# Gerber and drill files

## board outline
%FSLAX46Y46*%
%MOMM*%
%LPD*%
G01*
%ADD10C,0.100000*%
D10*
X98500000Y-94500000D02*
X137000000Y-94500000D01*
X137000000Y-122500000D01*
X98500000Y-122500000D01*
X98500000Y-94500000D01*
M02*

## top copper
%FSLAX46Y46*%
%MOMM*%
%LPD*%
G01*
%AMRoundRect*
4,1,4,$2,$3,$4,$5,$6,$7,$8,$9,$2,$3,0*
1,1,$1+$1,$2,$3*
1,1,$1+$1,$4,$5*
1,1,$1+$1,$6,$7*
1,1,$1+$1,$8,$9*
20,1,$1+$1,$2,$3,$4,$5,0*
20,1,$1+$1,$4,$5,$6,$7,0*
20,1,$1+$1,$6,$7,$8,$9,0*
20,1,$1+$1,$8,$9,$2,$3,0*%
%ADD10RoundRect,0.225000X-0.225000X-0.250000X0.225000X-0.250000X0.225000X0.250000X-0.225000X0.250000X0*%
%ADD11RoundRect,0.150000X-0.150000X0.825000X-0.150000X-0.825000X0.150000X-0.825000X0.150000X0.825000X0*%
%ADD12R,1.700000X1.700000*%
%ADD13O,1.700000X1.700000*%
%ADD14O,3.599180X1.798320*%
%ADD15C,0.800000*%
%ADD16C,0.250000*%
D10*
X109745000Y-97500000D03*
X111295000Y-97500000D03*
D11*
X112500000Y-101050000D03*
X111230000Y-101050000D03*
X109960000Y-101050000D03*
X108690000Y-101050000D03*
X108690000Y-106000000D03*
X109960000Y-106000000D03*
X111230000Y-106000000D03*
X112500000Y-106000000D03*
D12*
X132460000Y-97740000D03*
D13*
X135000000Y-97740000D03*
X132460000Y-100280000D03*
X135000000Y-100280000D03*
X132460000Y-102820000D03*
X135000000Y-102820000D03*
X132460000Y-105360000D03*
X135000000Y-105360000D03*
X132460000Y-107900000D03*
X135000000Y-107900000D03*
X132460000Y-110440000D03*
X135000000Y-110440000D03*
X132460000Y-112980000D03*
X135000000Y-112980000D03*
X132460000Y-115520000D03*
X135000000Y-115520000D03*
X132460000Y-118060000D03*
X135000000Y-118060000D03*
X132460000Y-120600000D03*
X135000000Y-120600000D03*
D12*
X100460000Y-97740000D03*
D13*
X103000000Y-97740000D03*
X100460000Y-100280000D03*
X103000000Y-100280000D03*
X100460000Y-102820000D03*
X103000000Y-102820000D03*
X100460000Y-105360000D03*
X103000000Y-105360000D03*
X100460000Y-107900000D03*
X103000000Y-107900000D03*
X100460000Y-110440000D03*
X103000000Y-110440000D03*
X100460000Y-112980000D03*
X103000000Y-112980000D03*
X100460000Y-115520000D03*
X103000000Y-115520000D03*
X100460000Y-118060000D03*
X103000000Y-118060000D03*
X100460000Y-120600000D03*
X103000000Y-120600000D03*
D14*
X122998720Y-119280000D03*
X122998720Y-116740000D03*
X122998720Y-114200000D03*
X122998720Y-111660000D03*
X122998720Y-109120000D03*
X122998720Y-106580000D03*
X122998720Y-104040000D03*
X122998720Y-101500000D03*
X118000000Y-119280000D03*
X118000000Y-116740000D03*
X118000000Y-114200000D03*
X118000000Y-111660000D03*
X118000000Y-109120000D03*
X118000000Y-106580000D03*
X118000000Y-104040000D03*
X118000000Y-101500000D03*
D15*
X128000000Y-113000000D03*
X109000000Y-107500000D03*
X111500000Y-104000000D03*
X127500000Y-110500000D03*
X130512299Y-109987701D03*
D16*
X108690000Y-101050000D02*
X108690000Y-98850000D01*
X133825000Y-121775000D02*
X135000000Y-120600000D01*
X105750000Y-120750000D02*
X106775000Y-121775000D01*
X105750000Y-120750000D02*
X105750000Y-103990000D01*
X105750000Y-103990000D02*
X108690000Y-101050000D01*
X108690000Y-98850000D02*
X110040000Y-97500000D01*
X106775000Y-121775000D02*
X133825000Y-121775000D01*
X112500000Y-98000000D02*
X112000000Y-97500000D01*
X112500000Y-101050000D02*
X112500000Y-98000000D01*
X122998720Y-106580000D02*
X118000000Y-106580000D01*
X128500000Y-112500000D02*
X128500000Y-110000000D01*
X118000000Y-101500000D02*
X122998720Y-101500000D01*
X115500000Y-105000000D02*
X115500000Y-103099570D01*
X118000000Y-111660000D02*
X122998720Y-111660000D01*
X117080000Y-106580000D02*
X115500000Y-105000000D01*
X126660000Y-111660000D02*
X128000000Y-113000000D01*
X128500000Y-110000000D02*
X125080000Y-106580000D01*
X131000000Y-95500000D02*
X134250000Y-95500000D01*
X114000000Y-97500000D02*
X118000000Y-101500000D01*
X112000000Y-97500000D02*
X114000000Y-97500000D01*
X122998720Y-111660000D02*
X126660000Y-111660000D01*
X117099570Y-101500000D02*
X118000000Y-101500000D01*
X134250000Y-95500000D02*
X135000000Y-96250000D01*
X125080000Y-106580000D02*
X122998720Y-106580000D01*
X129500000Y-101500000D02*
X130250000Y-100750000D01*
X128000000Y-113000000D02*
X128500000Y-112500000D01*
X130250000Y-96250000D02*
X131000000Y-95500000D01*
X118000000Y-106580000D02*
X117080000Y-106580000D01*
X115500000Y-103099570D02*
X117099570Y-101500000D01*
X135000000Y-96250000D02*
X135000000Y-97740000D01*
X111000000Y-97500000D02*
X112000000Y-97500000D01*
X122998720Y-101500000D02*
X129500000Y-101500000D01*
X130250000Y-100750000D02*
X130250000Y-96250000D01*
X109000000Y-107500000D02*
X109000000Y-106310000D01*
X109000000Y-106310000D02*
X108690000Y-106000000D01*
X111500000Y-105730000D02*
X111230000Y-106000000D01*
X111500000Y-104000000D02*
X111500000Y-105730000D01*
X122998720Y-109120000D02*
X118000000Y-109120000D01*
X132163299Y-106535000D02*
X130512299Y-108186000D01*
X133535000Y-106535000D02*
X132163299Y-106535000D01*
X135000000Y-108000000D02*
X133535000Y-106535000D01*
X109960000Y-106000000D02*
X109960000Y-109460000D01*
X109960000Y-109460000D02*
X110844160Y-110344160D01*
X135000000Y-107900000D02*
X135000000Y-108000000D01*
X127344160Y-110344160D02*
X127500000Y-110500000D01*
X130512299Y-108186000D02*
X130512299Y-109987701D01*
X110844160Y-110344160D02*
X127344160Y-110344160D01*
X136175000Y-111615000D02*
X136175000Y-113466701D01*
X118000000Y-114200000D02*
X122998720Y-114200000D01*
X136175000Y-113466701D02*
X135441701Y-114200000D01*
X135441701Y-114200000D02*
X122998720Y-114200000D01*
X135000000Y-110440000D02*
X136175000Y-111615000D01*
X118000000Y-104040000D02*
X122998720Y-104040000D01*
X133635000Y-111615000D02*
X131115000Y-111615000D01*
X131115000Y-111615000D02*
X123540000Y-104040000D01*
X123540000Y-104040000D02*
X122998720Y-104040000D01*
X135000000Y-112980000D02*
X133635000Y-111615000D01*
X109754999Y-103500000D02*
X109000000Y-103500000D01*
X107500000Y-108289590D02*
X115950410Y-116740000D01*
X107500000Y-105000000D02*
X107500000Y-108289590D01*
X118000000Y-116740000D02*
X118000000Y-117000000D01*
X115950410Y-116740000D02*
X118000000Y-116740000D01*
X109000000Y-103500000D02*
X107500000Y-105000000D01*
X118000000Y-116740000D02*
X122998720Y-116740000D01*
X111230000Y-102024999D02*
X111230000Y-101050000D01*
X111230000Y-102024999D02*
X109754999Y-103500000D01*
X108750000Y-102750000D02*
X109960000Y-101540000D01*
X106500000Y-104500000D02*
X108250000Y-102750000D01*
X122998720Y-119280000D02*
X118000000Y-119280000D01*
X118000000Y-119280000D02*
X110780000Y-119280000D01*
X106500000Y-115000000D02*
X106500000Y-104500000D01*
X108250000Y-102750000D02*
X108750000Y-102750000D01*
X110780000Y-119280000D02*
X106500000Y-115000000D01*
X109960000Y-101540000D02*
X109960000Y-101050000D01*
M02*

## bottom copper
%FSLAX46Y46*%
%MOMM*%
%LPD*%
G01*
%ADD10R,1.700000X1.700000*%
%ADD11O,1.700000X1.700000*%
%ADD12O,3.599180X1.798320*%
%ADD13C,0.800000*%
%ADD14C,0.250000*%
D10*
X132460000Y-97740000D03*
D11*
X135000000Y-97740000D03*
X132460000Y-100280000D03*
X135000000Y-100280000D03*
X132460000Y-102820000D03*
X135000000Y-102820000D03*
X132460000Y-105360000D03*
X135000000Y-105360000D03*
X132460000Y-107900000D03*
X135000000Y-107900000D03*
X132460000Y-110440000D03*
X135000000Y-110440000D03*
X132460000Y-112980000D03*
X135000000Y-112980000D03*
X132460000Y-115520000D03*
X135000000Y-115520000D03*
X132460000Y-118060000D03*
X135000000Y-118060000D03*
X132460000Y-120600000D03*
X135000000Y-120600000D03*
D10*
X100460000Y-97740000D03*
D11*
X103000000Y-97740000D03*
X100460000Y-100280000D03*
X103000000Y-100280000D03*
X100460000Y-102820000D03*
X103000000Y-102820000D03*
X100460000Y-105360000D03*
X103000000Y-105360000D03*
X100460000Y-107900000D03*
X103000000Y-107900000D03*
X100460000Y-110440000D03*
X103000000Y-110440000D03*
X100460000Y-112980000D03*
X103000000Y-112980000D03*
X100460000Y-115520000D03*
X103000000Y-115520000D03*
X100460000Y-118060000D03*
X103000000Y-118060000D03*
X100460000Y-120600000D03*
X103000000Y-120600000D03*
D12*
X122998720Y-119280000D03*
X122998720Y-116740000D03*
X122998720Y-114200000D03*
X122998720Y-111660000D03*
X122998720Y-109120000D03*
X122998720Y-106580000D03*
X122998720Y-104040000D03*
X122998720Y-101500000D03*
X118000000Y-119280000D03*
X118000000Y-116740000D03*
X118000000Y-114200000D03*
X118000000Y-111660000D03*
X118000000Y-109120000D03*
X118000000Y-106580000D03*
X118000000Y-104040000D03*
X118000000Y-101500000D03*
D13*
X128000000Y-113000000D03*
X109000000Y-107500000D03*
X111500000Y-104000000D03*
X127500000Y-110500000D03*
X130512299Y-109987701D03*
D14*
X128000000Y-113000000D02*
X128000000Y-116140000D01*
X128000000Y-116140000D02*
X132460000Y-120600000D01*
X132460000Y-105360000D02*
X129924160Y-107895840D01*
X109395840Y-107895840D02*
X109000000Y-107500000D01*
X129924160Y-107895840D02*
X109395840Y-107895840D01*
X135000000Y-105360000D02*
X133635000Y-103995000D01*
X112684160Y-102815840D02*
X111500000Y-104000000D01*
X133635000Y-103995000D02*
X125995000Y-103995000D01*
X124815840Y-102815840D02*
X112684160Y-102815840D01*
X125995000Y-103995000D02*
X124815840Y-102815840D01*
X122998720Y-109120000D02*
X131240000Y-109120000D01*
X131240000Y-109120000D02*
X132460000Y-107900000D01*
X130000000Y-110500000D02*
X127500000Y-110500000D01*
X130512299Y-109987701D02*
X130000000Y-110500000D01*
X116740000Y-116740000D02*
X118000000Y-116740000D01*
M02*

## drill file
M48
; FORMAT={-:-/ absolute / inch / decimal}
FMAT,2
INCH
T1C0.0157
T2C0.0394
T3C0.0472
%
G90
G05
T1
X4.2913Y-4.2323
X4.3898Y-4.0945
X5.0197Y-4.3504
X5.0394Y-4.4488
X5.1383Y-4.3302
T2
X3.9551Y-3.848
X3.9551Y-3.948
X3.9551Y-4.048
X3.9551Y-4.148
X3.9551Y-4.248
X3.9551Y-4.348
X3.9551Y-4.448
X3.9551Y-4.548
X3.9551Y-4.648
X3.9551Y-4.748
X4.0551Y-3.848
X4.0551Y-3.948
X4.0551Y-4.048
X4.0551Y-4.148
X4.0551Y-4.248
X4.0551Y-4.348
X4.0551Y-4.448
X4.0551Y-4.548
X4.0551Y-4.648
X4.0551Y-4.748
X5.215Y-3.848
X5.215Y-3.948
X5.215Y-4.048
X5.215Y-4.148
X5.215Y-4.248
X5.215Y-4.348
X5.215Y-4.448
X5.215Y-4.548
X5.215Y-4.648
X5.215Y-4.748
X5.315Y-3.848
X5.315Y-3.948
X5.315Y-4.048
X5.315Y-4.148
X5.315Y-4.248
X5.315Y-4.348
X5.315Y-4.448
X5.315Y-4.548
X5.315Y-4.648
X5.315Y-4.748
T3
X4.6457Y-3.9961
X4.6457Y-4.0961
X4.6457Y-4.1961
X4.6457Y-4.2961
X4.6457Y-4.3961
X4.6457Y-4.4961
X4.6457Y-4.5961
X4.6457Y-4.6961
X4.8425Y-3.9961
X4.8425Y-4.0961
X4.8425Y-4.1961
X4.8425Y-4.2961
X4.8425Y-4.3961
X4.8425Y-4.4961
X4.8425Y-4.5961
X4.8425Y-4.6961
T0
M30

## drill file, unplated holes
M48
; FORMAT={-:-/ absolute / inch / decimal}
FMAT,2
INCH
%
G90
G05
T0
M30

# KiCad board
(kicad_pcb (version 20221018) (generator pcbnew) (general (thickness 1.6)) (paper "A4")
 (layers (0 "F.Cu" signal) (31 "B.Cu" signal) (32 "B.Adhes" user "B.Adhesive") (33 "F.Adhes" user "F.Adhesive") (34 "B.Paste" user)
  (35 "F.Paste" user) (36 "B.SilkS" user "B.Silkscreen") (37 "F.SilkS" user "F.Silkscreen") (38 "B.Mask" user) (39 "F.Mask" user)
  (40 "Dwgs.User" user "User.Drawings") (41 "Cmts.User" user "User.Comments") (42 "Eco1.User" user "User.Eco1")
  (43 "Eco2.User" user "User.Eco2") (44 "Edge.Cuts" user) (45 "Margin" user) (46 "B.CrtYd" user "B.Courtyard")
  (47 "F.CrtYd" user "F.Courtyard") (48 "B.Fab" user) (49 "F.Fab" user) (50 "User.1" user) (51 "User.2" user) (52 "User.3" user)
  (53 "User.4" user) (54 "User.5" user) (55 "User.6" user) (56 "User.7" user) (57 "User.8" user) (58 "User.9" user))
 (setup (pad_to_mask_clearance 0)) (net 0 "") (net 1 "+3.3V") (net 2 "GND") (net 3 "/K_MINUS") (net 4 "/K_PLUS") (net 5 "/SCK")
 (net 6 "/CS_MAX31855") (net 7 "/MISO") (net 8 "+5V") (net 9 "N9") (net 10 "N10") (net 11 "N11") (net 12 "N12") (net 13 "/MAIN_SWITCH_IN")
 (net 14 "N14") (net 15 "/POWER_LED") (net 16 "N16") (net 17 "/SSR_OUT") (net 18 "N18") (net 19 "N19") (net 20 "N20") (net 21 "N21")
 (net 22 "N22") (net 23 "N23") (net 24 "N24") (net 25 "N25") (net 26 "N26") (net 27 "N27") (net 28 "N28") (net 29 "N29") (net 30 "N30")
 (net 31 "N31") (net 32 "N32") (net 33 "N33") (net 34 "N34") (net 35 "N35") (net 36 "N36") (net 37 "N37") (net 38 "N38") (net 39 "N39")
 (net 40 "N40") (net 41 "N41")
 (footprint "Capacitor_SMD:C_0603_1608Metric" (layer "F.Cu") (at 110.52 97.5)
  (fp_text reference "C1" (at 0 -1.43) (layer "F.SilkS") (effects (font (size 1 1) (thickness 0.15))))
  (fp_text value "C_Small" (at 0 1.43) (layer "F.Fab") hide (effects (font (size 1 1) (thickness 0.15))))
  (pad "1" smd roundrect (at -0.775 0) (size 0.9 0.95) (layers "F.Cu" "F.Paste" "F.Mask") (roundrect_rratio 0.25) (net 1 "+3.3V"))
  (pad "2" smd roundrect (at 0.775 0) (size 0.9 0.95) (layers "F.Cu" "F.Paste" "F.Mask") (roundrect_rratio 0.25) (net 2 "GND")))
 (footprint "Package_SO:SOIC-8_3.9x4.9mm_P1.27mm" (layer "F.Cu") (at 110.595 103.525 -90)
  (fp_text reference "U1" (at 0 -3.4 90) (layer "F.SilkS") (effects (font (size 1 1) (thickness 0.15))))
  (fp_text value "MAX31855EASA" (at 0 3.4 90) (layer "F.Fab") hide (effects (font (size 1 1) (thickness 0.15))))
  (pad "1" smd roundrect (at -2.475 -1.905 270) (size 1.95 0.6) (layers "F.Cu" "F.Paste" "F.Mask") (roundrect_rratio 0.25) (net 2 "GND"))
  (pad "2" smd roundrect (at -2.475 -0.635 270) (size 1.95 0.6) (layers "F.Cu" "F.Paste" "F.Mask") (roundrect_rratio 0.25)
   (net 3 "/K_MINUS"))
  (pad "3" smd roundrect (at -2.475 0.635 270) (size 1.95 0.6) (layers "F.Cu" "F.Paste" "F.Mask") (roundrect_rratio 0.25) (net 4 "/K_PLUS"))
  (pad "4" smd roundrect (at -2.475 1.905 270) (size 1.95 0.6) (layers "F.Cu" "F.Paste" "F.Mask") (roundrect_rratio 0.25) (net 1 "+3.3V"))
  (pad "5" smd roundrect (at 2.475 1.905 270) (size 1.95 0.6) (layers "F.Cu" "F.Paste" "F.Mask") (roundrect_rratio 0.25) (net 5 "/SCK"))
  (pad "6" smd roundrect (at 2.475 0.635 270) (size 1.95 0.6) (layers "F.Cu" "F.Paste" "F.Mask") (roundrect_rratio 0.25)
   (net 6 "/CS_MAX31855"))
  (pad "7" smd roundrect (at 2.475 -0.635 270) (size 1.95 0.6) (layers "F.Cu" "F.Paste" "F.Mask") (roundrect_rratio 0.25) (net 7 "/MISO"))
  (pad "8" smd roundrect (at 2.475 -1.905 270) (size 1.95 0.6) (layers "F.Cu" "F.Paste" "F.Mask") (roundrect_rratio 0.25)))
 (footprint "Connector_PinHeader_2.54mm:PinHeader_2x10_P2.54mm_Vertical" (layer "F.Cu") (at 132.46 97.74)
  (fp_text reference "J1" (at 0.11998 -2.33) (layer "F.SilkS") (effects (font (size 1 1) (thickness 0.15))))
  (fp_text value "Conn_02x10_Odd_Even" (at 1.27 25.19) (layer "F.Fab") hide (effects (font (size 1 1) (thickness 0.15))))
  (pad "1" thru_hole rect (at 0 0) (size 1.7 1.7) (drill 1) (layers "*.Cu" "*.Mask") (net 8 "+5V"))
  (pad "2" thru_hole oval (at 2.54 0) (size 1.7 1.7) (drill 1) (layers "*.Cu" "*.Mask") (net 2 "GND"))
  (pad "3" thru_hole oval (at 0 2.54) (size 1.7 1.7) (drill 1) (layers "*.Cu" "*.Mask") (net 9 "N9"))
  (pad "4" thru_hole oval (at 2.54 2.54) (size 1.7 1.7) (drill 1) (layers "*.Cu" "*.Mask") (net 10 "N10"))
  (pad "5" thru_hole oval (at 0 5.08) (size 1.7 1.7) (drill 1) (layers "*.Cu" "*.Mask") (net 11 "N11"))
  (pad "6" thru_hole oval (at 2.54 5.08) (size 1.7 1.7) (drill 1) (layers "*.Cu" "*.Mask") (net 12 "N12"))
  (pad "7" thru_hole oval (at 0 7.62) (size 1.7 1.7) (drill 1) (layers "*.Cu" "*.Mask") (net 5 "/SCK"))
  (pad "8" thru_hole oval (at 2.54 7.62) (size 1.7 1.7) (drill 1) (layers "*.Cu" "*.Mask") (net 7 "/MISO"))
  (pad "9" thru_hole oval (at 0 10.16) (size 1.7 1.7) (drill 1) (layers "*.Cu" "*.Mask") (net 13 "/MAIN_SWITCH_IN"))
  (pad "10" thru_hole oval (at 2.54 10.16) (size 1.7 1.7) (drill 1) (layers "*.Cu" "*.Mask") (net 6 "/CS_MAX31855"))
  (pad "11" thru_hole oval (at 0 12.7) (size 1.7 1.7) (drill 1) (layers "*.Cu" "*.Mask") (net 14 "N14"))
  (pad "12" thru_hole oval (at 2.54 12.7) (size 1.7 1.7) (drill 1) (layers "*.Cu" "*.Mask") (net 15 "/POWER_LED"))
  (pad "13" thru_hole oval (at 0 15.24) (size 1.7 1.7) (drill 1) (layers "*.Cu" "*.Mask") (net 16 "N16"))
  (pad "14" thru_hole oval (at 2.54 15.24) (size 1.7 1.7) (drill 1) (layers "*.Cu" "*.Mask") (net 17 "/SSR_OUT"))
  (pad "15" thru_hole oval (at 0 17.78) (size 1.7 1.7) (drill 1) (layers "*.Cu" "*.Mask") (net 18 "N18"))
  (pad "16" thru_hole oval (at 2.54 17.78) (size 1.7 1.7) (drill 1) (layers "*.Cu" "*.Mask") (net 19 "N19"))
  (pad "17" thru_hole oval (at 0 20.32) (size 1.7 1.7) (drill 1) (layers "*.Cu" "*.Mask") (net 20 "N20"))
  (pad "18" thru_hole oval (at 2.54 20.32) (size 1.7 1.7) (drill 1) (layers "*.Cu" "*.Mask") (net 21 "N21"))
  (pad "19" thru_hole oval (at 0 22.86) (size 1.7 1.7) (drill 1) (layers "*.Cu" "*.Mask") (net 2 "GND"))
  (pad "20" thru_hole oval (at 2.54 22.86) (size 1.7 1.7) (drill 1) (layers "*.Cu" "*.Mask") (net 1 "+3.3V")))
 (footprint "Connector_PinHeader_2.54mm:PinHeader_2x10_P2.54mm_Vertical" (layer "F.Cu") (at 100.46 97.74)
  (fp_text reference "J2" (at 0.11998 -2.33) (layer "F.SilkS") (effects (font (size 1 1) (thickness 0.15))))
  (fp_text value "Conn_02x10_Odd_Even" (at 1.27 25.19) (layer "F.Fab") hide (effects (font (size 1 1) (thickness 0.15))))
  (pad "1" thru_hole rect (at 0 0) (size 1.7 1.7) (drill 1) (layers "*.Cu" "*.Mask") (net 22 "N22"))
  (pad "2" thru_hole oval (at 2.54 0) (size 1.7 1.7) (drill 1) (layers "*.Cu" "*.Mask") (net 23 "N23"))
  (pad "3" thru_hole oval (at 0 2.54) (size 1.7 1.7) (drill 1) (layers "*.Cu" "*.Mask") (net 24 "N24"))
  (pad "4" thru_hole oval (at 2.54 2.54) (size 1.7 1.7) (drill 1) (layers "*.Cu" "*.Mask") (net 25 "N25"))
  (pad "5" thru_hole oval (at 0 5.08) (size 1.7 1.7) (drill 1) (layers "*.Cu" "*.Mask") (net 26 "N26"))
  (pad "6" thru_hole oval (at 2.54 5.08) (size 1.7 1.7) (drill 1) (layers "*.Cu" "*.Mask") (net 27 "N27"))
  (pad "7" thru_hole oval (at 0 7.62) (size 1.7 1.7) (drill 1) (layers "*.Cu" "*.Mask") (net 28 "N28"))
  (pad "8" thru_hole oval (at 2.54 7.62) (size 1.7 1.7) (drill 1) (layers "*.Cu" "*.Mask") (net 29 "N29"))
  (pad "9" thru_hole oval (at 0 10.16) (size 1.7 1.7) (drill 1) (layers "*.Cu" "*.Mask") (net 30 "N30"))
  (pad "10" thru_hole oval (at 2.54 10.16) (size 1.7 1.7) (drill 1) (layers "*.Cu" "*.Mask") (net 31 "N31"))
  (pad "11" thru_hole oval (at 0 12.7) (size 1.7 1.7) (drill 1) (layers "*.Cu" "*.Mask") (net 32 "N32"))
  (pad "12" thru_hole oval (at 2.54 12.7) (size 1.7 1.7) (drill 1) (layers "*.Cu" "*.Mask") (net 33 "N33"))
  (pad "13" thru_hole oval (at 0 15.24) (size 1.7 1.7) (drill 1) (layers "*.Cu" "*.Mask") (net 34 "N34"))
  (pad "14" thru_hole oval (at 2.54 15.24) (size 1.7 1.7) (drill 1) (layers "*.Cu" "*.Mask") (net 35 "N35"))
  (pad "15" thru_hole oval (at 0 17.78) (size 1.7 1.7) (drill 1) (layers "*.Cu" "*.Mask") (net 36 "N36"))
  (pad "16" thru_hole oval (at 2.54 17.78) (size 1.7 1.7) (drill 1) (layers "*.Cu" "*.Mask") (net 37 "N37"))
  (pad "17" thru_hole oval (at 0 20.32) (size 1.7 1.7) (drill 1) (layers "*.Cu" "*.Mask") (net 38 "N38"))
  (pad "18" thru_hole oval (at 2.54 20.32) (size 1.7 1.7) (drill 1) (layers "*.Cu" "*.Mask") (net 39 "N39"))
  (pad "19" thru_hole oval (at 0 22.86) (size 1.7 1.7) (drill 1) (layers "*.Cu" "*.Mask") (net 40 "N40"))
  (pad "20" thru_hole oval (at 2.54 22.86) (size 1.7 1.7) (drill 1) (layers "*.Cu" "*.Mask") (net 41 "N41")))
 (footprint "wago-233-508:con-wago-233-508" (layer "B.Cu") (at 120.49936 110.39 90)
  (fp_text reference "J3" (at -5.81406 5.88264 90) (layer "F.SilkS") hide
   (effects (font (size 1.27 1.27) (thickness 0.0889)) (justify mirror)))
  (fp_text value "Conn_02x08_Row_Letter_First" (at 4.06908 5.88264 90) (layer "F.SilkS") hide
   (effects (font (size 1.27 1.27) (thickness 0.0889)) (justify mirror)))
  (pad "a1" thru_hole oval (at -8.89 2.49936 90) (size 1.79832 3.59918) (drill 1.19888) (layers "*.Cu" "B.Paste" "B.Mask") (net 4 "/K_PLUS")
   (thermal_bridge_angle 45))
  (pad "a2" thru_hole oval (at -6.35 2.49936 90) (size 1.79832 3.59918) (drill 1.19888) (layers "*.Cu" "B.Paste" "B.Mask")
   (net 3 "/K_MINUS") (thermal_bridge_angle 45))
  (pad "a3" thru_hole oval (at -3.81 2.49936 90) (size 1.79832 3.59918) (drill 1.19888) (layers "*.Cu" "B.Paste" "B.Mask")
   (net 15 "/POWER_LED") (thermal_bridge_angle 45))
  (pad "a4" thru_hole oval (at -1.27 2.49936 90) (size 1.79832 3.59918) (drill 1.19888) (layers "*.Cu" "B.Paste" "B.Mask") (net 2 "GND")
   (thermal_bridge_angle 45))
  (pad "a5" thru_hole oval (at 1.27 2.49936 90) (size 1.79832 3.59918) (drill 1.19888) (layers "*.Cu" "B.Paste" "B.Mask")
   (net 13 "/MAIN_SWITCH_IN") (thermal_bridge_angle 45))
  (pad "a6" thru_hole oval (at 3.81 2.49936 90) (size 1.79832 3.59918) (drill 1.19888) (layers "*.Cu" "B.Paste" "B.Mask") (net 2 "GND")
   (thermal_bridge_angle 45))
  (pad "a7" thru_hole oval (at 6.35 2.49936 90) (size 1.79832 3.59918) (drill 1.19888) (layers "*.Cu" "B.Paste" "B.Mask")
   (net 17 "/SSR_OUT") (thermal_bridge_angle 45))
  (pad "a8" thru_hole oval (at 8.89 2.49936 90) (size 1.79832 3.59918) (drill 1.19888) (layers "*.Cu" "B.Paste" "B.Mask") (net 2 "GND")
   (thermal_bridge_angle 45))
  (pad "b1" thru_hole oval (at -8.89 -2.49936 90) (size 1.79832 3.59918) (drill 1.19888) (layers "*.Cu" "B.Paste" "B.Mask")
   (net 4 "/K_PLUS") (thermal_bridge_angle 45))
  (pad "b2" thru_hole oval (at -6.35 -2.49936 90) (size 1.79832 3.59918) (drill 1.19888) (layers "*.Cu" "B.Paste" "B.Mask")
   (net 3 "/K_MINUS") (thermal_bridge_angle 45))
  (pad "b3" thru_hole oval (at -3.81 -2.49936 90) (size 1.79832 3.59918) (drill 1.19888) (layers "*.Cu" "B.Paste" "B.Mask")
   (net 15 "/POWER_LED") (thermal_bridge_angle 45))
  (pad "b4" thru_hole oval (at -1.27 -2.49936 90) (size 1.79832 3.59918) (drill 1.19888) (layers "*.Cu" "B.Paste" "B.Mask") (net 2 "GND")
   (thermal_bridge_angle 45))
  (pad "b5" thru_hole oval (at 1.27 -2.49936 90) (size 1.79832 3.59918) (drill 1.19888) (layers "*.Cu" "B.Paste" "B.Mask")
   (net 13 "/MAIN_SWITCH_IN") (thermal_bridge_angle 45))
  (pad "b6" thru_hole oval (at 3.81 -2.49936 90) (size 1.79832 3.59918) (drill 1.19888) (layers "*.Cu" "B.Paste" "B.Mask") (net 2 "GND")
   (thermal_bridge_angle 45))
  (pad "b7" thru_hole oval (at 6.35 -2.49936 90) (size 1.79832 3.59918) (drill 1.19888) (layers "*.Cu" "B.Paste" "B.Mask")
   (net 17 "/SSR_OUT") (thermal_bridge_angle 45))
  (pad "b8" thru_hole oval (at 8.89 -2.49936 90) (size 1.79832 3.59918) (drill 1.19888) (layers "*.Cu" "B.Paste" "B.Mask") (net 2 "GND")
   (thermal_bridge_angle 45)))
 (gr_rect (start 98.5 94.5) (end 137 122.5) (stroke (width 0.1) (type default)) (fill none) (layer "Edge.Cuts"))
 (segment (start 108.69 101.05) (end 108.69 98.85) (width 0.25) (layer "F.Cu") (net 1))
 (segment (start 133.825 121.775) (end 135 120.6) (width 0.25) (layer "F.Cu") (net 1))
 (segment (start 105.75 120.75) (end 106.775 121.775) (width 0.25) (layer "F.Cu") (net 1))
 (segment (start 105.75 120.75) (end 105.75 103.99) (width 0.25) (layer "F.Cu") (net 1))
 (segment (start 105.75 103.99) (end 108.69 101.05) (width 0.25) (layer "F.Cu") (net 1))
 (segment (start 108.69 98.85) (end 110.04 97.5) (width 0.25) (layer "F.Cu") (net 1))
 (segment (start 106.775 121.775) (end 133.825 121.775) (width 0.25) (layer "F.Cu") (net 1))
 (segment (start 112.5 98) (end 112 97.5) (width 0.25) (layer "F.Cu") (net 2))
 (segment (start 112.5 101.05) (end 112.5 98) (width 0.25) (layer "F.Cu") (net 2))
 (segment (start 122.99872 106.58) (end 118 106.58) (width 0.25) (layer "F.Cu") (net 2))
 (segment (start 128.5 112.5) (end 128.5 110) (width 0.25) (layer "F.Cu") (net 2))
 (segment (start 118 101.5) (end 122.99872 101.5) (width 0.25) (layer "F.Cu") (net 2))
 (segment (start 115.5 105) (end 115.5 103.09957) (width 0.25) (layer "F.Cu") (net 2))
 (segment (start 118 111.66) (end 122.99872 111.66) (width 0.25) (layer "F.Cu") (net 2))
 (segment (start 117.08 106.58) (end 115.5 105) (width 0.25) (layer "F.Cu") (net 2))
 (segment (start 126.66 111.66) (end 128 113) (width 0.25) (layer "F.Cu") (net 2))
 (segment (start 128.5 110) (end 125.08 106.58) (width 0.25) (layer "F.Cu") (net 2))
 (segment (start 131 95.5) (end 134.25 95.5) (width 0.25) (layer "F.Cu") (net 2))
 (segment (start 114 97.5) (end 118 101.5) (width 0.25) (layer "F.Cu") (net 2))
 (segment (start 112 97.5) (end 114 97.5) (width 0.25) (layer "F.Cu") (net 2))
 (segment (start 122.99872 111.66) (end 126.66 111.66) (width 0.25) (layer "F.Cu") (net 2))
 (segment (start 117.09957 101.5) (end 118 101.5) (width 0.25) (layer "F.Cu") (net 2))
 (segment (start 134.25 95.5) (end 135 96.25) (width 0.25) (layer "F.Cu") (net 2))
 (segment (start 125.08 106.58) (end 122.99872 106.58) (width 0.25) (layer "F.Cu") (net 2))
 (segment (start 129.5 101.5) (end 130.25 100.75) (width 0.25) (layer "F.Cu") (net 2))
 (segment (start 128 113) (end 128.5 112.5) (width 0.25) (layer "F.Cu") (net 2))
 (segment (start 130.25 96.25) (end 131 95.5) (width 0.25) (layer "F.Cu") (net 2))
 (segment (start 118 106.58) (end 117.08 106.58) (width 0.25) (layer "F.Cu") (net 2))
 (segment (start 115.5 103.09957) (end 117.09957 101.5) (width 0.25) (layer "F.Cu") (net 2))
 (segment (start 135 96.25) (end 135 97.74) (width 0.25) (layer "F.Cu") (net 2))
 (segment (start 111 97.5) (end 112 97.5) (width 0.25) (layer "F.Cu") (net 2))
 (segment (start 122.99872 101.5) (end 129.5 101.5) (width 0.25) (layer "F.Cu") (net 2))
 (segment (start 130.25 100.75) (end 130.25 96.25) (width 0.25) (layer "F.Cu") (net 2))
 (via (at 128 113) (size 0.8) (drill 0.4) (layers "F.Cu" "B.Cu") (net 2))
 (segment (start 128 113) (end 128 116.14) (width 0.25) (layer "B.Cu") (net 2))
 (segment (start 128 116.14) (end 132.46 120.6) (width 0.25) (layer "B.Cu") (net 2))
 (segment (start 109 107.5) (end 109 106.31) (width 0.25) (layer "F.Cu") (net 5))
 (segment (start 109 106.31) (end 108.69 106) (width 0.25) (layer "F.Cu") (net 5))
 (via (at 109 107.5) (size 0.8) (drill 0.4) (layers "F.Cu" "B.Cu") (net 5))
 (segment (start 132.46 105.36) (end 129.92416 107.89584) (width 0.25) (layer "B.Cu") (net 5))
 (segment (start 109.39584 107.89584) (end 109 107.5) (width 0.25) (layer "B.Cu") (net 5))
 (segment (start 129.92416 107.89584) (end 109.39584 107.89584) (width 0.25) (layer "B.Cu") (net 5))
 (segment (start 111.5 105.73) (end 111.23 106) (width 0.25) (layer "F.Cu") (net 7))
 (segment (start 111.5 104) (end 111.5 105.73) (width 0.25) (layer "F.Cu") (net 7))
 (via (at 111.5 104) (size 0.8) (drill 0.4) (layers "F.Cu" "B.Cu") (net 7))
 (segment (start 135 105.36) (end 133.635 103.995) (width 0.25) (layer "B.Cu") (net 7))
 (segment (start 112.68416 102.81584) (end 111.5 104) (width 0.25) (layer "B.Cu") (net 7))
 (segment (start 133.635 103.995) (end 125.995 103.995) (width 0.25) (layer "B.Cu") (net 7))
 (segment (start 124.81584 102.81584) (end 112.68416 102.81584) (width 0.25) (layer "B.Cu") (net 7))
 (segment (start 125.995 103.995) (end 124.81584 102.81584) (width 0.25) (layer "B.Cu") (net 7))
 (segment (start 122.99872 109.12) (end 118 109.12) (width 0.25) (layer "F.Cu") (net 13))
 (segment (start 122.99872 109.12) (end 131.24 109.12) (width 0.25) (layer "B.Cu") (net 13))
 (segment (start 131.24 109.12) (end 132.46 107.9) (width 0.25) (layer "B.Cu") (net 13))
 (segment (start 132.163299 106.535) (end 130.512299 108.186) (width 0.25) (layer "F.Cu") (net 6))
 (segment (start 133.535 106.535) (end 132.163299 106.535) (width 0.25) (layer "F.Cu") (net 6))
 (segment (start 135 108) (end 133.535 106.535) (width 0.25) (layer "F.Cu") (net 6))
 (segment (start 109.96 106) (end 109.96 109.46) (width 0.25) (layer "F.Cu") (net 6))
 (segment (start 109.96 109.46) (end 110.84416 110.34416) (width 0.25) (layer "F.Cu") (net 6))
 (segment (start 135 107.9) (end 135 108) (width 0.25) (layer "F.Cu") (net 6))
 (segment (start 127.34416 110.34416) (end 127.5 110.5) (width 0.25) (layer "F.Cu") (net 6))
 (segment (start 130.512299 108.186) (end 130.512299 109.987701) (width 0.25) (layer "F.Cu") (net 6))
 (segment (start 110.84416 110.34416) (end 127.34416 110.34416) (width 0.25) (layer "F.Cu") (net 6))
 (via (at 127.5 110.5) (size 0.8) (drill 0.4) (layers "F.Cu" "B.Cu") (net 6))
 (via (at 130.512299 109.987701) (size 0.8) (drill 0.4) (layers "F.Cu" "B.Cu") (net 6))
 (segment (start 130 110.5) (end 127.5 110.5) (width 0.25) (layer "B.Cu") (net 6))
 (segment (start 130.512299 109.987701) (end 130 110.5) (width 0.25) (layer "B.Cu") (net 6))
 (segment (start 136.175 111.615) (end 136.175 113.466701) (width 0.25) (layer "F.Cu") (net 15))
 (segment (start 118 114.2) (end 122.99872 114.2) (width 0.25) (layer "F.Cu") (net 15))
 (segment (start 136.175 113.466701) (end 135.441701 114.2) (width 0.25) (layer "F.Cu") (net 15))
 (segment (start 135.441701 114.2) (end 122.99872 114.2) (width 0.25) (layer "F.Cu") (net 15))
 (segment (start 135 110.44) (end 136.175 111.615) (width 0.25) (layer "F.Cu") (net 15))
 (segment (start 118 104.04) (end 122.99872 104.04) (width 0.25) (layer "F.Cu") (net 17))
 (segment (start 133.635 111.615) (end 131.115 111.615) (width 0.25) (layer "F.Cu") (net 17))
 (segment (start 131.115 111.615) (end 123.54 104.04) (width 0.25) (layer "F.Cu") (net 17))
 (segment (start 123.54 104.04) (end 122.99872 104.04) (width 0.25) (layer "F.Cu") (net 17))
 (segment (start 135 112.98) (end 133.635 111.615) (width 0.25) (layer "F.Cu") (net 17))
 (segment (start 109.754999 103.5) (end 109 103.5) (width 0.25) (layer "F.Cu") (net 3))
 (segment (start 107.5 108.28959) (end 115.95041 116.74) (width 0.25) (layer "F.Cu") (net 3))
 (segment (start 107.5 105) (end 107.5 108.28959) (width 0.25) (layer "F.Cu") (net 3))
 (segment (start 118 116.74) (end 118 117) (width 0.25) (layer "F.Cu") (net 3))
 (segment (start 115.95041 116.74) (end 118 116.74) (width 0.25) (layer "F.Cu") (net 3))
 (segment (start 109 103.5) (end 107.5 105) (width 0.25) (layer "F.Cu") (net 3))
 (segment (start 118 116.74) (end 122.99872 116.74) (width 0.25) (layer "F.Cu") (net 3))
 (segment (start 111.23 102.024999) (end 111.23 101.05) (width 0.25) (layer "F.Cu") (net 3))
 (segment (start 111.23 102.024999) (end 109.754999 103.5) (width 0.25) (layer "F.Cu") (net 3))
 (segment (start 116.74 116.74) (end 118 116.74) (width 0.25) (layer "B.Cu") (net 3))
 (segment (start 108.75 102.75) (end 109.96 101.54) (width 0.25) (layer "F.Cu") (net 4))
 (segment (start 106.5 104.5) (end 108.25 102.75) (width 0.25) (layer "F.Cu") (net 4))
 (segment (start 122.99872 119.28) (end 118 119.28) (width 0.25) (layer "F.Cu") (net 4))
 (segment (start 118 119.28) (end 110.78 119.28) (width 0.25) (layer "F.Cu") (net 4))
 (segment (start 106.5 115) (end 106.5 104.5) (width 0.25) (layer "F.Cu") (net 4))
 (segment (start 108.25 102.75) (end 108.75 102.75) (width 0.25) (layer "F.Cu") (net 4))
 (segment (start 110.78 119.28) (end 106.5 115) (width 0.25) (layer "F.Cu") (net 4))
 (segment (start 109.96 101.54) (end 109.96 101.05) (width 0.25) (layer "F.Cu") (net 4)))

